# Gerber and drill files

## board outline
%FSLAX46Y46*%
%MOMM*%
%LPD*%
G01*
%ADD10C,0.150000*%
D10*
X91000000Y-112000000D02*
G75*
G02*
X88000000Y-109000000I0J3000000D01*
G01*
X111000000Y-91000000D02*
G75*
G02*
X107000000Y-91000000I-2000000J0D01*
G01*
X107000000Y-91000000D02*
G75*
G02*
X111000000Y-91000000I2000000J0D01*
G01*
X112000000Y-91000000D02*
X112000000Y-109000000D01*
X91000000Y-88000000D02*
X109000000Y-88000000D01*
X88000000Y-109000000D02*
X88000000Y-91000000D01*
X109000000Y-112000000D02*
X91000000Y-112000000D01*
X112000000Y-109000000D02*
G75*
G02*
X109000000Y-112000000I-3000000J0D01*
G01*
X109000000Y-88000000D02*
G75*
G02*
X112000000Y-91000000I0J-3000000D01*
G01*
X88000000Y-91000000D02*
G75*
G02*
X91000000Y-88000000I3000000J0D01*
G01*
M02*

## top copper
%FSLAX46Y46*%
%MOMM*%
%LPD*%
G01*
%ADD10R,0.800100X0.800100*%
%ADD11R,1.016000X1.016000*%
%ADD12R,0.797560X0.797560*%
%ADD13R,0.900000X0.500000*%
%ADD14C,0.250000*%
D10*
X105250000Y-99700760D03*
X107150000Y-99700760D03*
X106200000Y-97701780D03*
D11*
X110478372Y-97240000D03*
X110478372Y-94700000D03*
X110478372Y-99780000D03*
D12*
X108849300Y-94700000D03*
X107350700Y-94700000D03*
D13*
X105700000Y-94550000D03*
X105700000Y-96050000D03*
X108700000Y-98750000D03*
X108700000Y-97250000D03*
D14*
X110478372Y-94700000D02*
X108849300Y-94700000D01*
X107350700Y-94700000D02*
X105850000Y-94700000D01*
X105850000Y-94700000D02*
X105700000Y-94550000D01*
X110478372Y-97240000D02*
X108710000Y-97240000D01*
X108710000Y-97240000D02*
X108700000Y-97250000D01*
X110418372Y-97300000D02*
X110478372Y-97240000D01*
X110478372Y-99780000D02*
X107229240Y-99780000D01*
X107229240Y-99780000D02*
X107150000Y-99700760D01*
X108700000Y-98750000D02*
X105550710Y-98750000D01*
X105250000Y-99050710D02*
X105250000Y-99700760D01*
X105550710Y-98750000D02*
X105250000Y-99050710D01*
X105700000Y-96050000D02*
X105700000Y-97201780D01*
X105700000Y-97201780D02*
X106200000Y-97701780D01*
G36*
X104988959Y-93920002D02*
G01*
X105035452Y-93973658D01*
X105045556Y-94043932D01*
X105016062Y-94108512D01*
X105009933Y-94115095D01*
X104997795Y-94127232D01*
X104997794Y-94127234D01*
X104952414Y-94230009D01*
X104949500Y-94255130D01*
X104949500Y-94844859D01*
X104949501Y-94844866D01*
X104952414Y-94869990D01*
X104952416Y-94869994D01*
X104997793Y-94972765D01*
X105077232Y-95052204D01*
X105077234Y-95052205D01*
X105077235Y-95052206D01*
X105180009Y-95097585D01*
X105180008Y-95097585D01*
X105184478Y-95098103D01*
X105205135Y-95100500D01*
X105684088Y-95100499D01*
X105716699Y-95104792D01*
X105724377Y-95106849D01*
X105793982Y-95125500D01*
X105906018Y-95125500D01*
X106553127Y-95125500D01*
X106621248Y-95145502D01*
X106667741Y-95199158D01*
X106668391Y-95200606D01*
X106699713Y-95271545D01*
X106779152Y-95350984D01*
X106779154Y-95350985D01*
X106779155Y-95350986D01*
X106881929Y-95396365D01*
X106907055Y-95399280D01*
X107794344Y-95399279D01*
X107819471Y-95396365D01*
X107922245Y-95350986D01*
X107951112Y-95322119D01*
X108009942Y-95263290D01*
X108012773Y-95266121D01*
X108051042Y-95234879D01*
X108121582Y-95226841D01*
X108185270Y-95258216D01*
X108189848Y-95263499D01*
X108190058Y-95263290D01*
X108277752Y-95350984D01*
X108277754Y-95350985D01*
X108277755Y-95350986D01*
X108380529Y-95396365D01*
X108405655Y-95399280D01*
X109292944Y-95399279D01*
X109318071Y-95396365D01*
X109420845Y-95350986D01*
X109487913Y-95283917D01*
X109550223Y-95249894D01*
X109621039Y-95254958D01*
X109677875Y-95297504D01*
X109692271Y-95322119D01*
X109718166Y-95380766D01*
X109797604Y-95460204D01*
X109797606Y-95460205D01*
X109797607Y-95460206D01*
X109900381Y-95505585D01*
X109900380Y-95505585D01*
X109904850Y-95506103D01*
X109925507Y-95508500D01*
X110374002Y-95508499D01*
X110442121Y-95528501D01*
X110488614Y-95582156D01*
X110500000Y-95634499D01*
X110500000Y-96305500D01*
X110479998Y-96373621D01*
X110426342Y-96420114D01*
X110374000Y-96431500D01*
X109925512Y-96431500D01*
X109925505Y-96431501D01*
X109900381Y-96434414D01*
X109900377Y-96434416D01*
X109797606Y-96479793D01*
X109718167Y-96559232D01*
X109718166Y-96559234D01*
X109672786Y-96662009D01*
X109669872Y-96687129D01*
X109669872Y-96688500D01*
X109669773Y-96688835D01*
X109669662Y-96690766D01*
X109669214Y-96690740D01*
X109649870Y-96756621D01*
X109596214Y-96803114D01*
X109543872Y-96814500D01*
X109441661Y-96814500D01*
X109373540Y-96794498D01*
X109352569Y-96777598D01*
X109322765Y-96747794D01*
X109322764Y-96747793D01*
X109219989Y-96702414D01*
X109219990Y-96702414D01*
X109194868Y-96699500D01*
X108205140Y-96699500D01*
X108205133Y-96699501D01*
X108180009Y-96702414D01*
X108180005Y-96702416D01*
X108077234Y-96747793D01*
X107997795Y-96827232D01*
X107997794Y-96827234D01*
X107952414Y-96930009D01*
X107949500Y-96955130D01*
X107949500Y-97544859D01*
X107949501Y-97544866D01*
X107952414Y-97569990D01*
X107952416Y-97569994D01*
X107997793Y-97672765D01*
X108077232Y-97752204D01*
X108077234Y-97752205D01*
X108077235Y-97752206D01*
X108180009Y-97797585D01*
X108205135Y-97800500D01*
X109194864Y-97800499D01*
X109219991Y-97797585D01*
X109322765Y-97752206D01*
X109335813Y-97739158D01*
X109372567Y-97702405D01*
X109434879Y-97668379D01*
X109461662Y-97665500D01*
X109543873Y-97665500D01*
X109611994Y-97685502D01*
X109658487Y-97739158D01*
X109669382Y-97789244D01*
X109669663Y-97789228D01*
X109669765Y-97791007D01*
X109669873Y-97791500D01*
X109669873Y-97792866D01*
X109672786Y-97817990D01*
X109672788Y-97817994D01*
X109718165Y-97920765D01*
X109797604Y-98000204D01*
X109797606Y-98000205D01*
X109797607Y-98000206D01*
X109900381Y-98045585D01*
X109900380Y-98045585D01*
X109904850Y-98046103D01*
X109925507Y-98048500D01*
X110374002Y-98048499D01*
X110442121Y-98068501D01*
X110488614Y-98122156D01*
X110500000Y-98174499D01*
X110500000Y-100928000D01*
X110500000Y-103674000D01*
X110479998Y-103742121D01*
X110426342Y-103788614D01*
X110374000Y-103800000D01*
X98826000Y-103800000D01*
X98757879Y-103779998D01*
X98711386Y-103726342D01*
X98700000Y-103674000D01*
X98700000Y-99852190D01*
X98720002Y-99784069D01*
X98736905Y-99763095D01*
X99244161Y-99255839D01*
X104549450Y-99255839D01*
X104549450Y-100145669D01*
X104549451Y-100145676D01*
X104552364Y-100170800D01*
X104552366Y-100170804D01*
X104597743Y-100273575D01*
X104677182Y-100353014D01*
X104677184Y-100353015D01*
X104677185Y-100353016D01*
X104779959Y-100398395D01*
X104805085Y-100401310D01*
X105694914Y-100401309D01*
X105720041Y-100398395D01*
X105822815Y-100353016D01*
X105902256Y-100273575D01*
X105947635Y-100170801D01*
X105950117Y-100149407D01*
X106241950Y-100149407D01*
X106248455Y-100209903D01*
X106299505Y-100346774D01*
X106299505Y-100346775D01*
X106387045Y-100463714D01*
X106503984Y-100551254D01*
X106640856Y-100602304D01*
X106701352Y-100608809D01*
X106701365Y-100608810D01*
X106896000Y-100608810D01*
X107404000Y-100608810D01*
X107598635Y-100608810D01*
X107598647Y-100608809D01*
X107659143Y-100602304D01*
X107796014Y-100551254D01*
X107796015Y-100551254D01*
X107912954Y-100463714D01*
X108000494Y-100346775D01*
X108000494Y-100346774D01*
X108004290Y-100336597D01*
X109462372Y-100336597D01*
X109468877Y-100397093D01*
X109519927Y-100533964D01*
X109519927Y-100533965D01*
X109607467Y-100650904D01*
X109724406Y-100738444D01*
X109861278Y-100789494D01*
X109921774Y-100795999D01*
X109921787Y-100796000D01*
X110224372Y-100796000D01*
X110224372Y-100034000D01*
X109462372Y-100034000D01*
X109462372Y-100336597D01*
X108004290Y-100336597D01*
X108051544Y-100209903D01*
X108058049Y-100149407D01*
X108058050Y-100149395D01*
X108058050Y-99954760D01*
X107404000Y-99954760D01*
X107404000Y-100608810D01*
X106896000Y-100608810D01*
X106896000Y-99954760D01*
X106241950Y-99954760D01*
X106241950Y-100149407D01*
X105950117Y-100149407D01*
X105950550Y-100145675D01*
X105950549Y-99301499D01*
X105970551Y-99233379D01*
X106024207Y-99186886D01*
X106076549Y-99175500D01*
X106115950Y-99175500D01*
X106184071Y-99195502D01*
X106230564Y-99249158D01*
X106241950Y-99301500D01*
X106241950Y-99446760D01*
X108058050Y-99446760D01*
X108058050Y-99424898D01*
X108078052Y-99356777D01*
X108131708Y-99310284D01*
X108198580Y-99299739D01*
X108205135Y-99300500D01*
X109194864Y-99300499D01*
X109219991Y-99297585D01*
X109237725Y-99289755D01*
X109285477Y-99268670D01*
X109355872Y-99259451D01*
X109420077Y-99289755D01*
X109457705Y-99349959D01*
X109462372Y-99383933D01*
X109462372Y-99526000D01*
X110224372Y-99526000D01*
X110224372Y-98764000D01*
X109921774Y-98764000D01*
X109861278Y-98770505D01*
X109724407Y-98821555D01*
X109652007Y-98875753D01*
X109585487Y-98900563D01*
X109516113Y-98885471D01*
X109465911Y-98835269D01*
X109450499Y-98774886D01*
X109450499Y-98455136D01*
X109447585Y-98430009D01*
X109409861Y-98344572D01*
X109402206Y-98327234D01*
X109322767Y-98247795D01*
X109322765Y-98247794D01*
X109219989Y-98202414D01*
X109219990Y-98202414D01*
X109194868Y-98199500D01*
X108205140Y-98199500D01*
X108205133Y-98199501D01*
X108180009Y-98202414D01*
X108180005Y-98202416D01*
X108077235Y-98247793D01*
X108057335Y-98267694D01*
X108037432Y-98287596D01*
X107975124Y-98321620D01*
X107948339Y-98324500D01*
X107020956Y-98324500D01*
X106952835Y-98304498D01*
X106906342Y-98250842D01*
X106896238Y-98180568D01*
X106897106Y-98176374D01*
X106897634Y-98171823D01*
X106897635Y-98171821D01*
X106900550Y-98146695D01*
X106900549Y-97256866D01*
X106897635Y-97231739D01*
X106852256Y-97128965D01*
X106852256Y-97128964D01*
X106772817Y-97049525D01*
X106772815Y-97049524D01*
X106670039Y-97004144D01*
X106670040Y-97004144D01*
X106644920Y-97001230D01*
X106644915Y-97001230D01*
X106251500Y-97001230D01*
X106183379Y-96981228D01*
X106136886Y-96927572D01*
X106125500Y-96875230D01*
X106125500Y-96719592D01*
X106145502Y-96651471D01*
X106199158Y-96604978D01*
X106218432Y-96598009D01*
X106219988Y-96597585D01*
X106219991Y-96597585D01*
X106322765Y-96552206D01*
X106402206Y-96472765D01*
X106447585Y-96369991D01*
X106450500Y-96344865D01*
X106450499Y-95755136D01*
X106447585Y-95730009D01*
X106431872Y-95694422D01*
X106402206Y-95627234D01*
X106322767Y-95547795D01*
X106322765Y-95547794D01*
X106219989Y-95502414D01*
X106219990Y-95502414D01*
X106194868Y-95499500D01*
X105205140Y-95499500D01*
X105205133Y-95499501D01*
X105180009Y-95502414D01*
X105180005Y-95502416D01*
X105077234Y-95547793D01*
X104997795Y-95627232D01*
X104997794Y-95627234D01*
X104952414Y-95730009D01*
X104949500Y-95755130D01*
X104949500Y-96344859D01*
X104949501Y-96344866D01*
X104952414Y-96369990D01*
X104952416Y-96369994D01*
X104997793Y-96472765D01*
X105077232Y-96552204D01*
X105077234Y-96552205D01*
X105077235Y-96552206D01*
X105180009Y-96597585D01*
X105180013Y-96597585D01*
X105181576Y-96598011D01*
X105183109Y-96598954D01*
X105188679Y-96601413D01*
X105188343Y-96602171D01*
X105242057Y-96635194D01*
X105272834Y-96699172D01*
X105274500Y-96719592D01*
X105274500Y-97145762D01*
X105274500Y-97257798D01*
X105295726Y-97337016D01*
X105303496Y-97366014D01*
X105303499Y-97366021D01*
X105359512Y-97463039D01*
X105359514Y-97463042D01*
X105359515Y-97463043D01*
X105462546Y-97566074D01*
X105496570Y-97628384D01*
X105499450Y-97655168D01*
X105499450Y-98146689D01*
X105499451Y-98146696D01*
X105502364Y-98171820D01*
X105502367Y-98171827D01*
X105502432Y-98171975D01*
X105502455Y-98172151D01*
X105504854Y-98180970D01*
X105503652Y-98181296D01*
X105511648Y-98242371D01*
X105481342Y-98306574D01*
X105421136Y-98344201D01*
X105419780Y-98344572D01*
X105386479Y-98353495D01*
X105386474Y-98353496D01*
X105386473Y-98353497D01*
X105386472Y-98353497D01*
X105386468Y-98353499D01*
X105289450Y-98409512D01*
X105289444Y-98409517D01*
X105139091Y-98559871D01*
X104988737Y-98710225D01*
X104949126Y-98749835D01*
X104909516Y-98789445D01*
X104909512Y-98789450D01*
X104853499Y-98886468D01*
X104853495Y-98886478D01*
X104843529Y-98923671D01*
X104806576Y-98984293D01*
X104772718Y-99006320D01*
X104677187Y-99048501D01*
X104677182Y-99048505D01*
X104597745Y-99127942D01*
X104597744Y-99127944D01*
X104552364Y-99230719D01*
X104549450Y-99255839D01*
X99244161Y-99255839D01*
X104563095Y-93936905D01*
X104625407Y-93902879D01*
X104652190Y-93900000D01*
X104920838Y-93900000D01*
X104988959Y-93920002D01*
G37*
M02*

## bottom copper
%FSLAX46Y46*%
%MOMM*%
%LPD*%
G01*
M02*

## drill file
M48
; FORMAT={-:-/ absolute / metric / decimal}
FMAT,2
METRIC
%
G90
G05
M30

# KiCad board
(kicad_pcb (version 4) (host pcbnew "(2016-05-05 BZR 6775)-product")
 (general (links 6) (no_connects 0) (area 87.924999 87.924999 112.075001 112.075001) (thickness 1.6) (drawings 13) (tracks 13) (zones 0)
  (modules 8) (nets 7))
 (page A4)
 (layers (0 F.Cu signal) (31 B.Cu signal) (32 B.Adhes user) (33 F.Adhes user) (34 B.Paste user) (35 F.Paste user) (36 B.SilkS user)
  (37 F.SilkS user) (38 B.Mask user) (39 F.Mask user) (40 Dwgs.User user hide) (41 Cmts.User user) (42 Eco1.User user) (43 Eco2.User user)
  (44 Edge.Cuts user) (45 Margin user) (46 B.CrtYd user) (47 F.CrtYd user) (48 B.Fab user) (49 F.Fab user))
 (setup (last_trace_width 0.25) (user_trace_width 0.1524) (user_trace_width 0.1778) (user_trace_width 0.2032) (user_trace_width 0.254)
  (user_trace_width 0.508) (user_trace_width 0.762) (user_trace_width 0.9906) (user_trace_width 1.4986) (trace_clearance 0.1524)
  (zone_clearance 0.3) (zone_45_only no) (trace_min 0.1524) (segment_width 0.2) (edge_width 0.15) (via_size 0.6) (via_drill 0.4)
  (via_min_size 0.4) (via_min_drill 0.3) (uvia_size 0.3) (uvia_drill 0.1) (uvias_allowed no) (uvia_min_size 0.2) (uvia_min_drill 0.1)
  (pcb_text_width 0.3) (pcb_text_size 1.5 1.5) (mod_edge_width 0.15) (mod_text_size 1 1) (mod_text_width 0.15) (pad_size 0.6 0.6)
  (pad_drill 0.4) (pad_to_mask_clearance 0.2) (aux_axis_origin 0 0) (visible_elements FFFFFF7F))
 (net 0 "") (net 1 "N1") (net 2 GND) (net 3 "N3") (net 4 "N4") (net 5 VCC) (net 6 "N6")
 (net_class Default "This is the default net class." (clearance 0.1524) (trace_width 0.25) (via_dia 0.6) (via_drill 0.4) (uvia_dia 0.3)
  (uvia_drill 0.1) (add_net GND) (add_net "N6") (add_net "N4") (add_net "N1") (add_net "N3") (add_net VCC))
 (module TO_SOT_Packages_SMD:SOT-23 (layer F.Cu) (at 106.2 98.7)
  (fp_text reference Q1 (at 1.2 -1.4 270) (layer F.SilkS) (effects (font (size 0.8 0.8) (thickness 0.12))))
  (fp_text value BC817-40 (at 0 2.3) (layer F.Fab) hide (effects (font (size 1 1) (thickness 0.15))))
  (pad 1 smd rect (at -0.95 1.00076) (size 0.8001 0.8001) (layers F.Cu F.Paste F.Mask) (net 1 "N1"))
  (pad 2 smd rect (at 0.95 1.00076) (size 0.8001 0.8001) (layers F.Cu F.Paste F.Mask) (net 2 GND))
  (pad 3 smd rect (at 0 -0.99822) (size 0.8001 0.8001) (layers F.Cu F.Paste F.Mask) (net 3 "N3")))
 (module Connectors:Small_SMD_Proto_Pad (layer F.Cu) (at 110.478372 97.24 180)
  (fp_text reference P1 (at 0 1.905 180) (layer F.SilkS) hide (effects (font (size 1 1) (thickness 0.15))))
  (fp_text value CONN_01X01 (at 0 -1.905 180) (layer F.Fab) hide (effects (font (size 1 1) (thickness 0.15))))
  (pad 1 smd rect (at 0 0 180) (size 1.016 1.016) (layers F.Cu F.Paste F.Mask) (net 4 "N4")))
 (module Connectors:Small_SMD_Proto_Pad (layer F.Cu) (at 110.478372 94.7 180)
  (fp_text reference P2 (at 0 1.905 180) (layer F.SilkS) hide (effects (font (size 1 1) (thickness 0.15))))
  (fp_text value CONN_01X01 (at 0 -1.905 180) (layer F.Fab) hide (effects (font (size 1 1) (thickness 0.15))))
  (pad 1 smd rect (at 0 0 180) (size 1.016 1.016) (layers F.Cu F.Paste F.Mask) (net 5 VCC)))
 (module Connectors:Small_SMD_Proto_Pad (layer F.Cu) (at 110.478372 99.78 180)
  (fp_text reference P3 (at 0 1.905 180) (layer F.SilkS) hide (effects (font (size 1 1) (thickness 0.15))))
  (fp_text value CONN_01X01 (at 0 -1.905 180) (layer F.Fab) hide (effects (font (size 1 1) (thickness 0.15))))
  (pad 1 smd rect (at 0 0 180) (size 1.016 1.016) (layers F.Cu F.Paste F.Mask) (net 2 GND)))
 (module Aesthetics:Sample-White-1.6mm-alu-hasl (layer F.Cu) (at 99.978372 102.6)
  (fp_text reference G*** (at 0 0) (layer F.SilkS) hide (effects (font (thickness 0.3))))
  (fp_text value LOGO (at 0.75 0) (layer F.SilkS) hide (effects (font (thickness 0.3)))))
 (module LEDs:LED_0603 (layer F.Cu) (at 108.1 94.7)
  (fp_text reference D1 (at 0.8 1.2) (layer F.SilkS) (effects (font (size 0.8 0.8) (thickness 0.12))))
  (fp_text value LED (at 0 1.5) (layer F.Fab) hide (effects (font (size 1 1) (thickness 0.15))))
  (pad 2 smd rect (at 0.7493 0 180) (size 0.79756 0.79756) (layers F.Cu F.Paste F.Mask) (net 5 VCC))
  (pad 1 smd rect (at -0.7493 0 180) (size 0.79756 0.79756) (layers F.Cu F.Paste F.Mask) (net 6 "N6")))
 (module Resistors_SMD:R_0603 (layer F.Cu) (at 105.7 95.3 270)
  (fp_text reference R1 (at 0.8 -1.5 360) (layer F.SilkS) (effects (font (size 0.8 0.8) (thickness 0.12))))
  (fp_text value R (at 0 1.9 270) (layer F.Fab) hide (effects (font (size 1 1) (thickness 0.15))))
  (pad 1 smd rect (at -0.75 0 270) (size 0.5 0.9) (layers F.Cu F.Paste F.Mask) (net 6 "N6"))
  (pad 2 smd rect (at 0.75 0 270) (size 0.5 0.9) (layers F.Cu F.Paste F.Mask) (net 3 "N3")))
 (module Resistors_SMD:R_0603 (layer F.Cu) (at 108.7 98 90)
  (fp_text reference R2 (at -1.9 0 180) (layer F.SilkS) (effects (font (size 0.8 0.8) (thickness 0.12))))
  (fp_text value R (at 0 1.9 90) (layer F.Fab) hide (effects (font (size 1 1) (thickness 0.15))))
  (pad 1 smd rect (at -0.75 0 90) (size 0.5 0.9) (layers F.Cu F.Paste F.Mask) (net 1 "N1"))
  (pad 2 smd rect (at 0.75 0 90) (size 0.5 0.9) (layers F.Cu F.Paste F.Mask) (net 4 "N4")))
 (gr_arc (start 91 109) (end 91 112) (angle 90) (layer Edge.Cuts) (width 0.15))
 (gr_circle (center 109 91) (end 111 91) (layer Edge.Cuts) (width 0.15))
 (gr_line (start 112 91) (end 112 109) (layer Edge.Cuts) (width 0.15))
 (gr_line (start 91 88) (end 109 88) (layer Edge.Cuts) (width 0.15))
 (gr_line (start 88 109) (end 88 91) (layer Edge.Cuts) (width 0.15))
 (gr_line (start 109 112) (end 91 112) (layer Edge.Cuts) (width 0.15))
 (gr_arc (start 109 109) (end 112 109) (angle 90) (layer Edge.Cuts) (width 0.15))
 (gr_arc (start 109 91) (end 109 88) (angle 90) (layer Edge.Cuts) (width 0.15))
 (gr_arc (start 91 91) (end 88 91) (angle 90) (layer Edge.Cuts) (width 0.15))
 (segment (start 110.478372 94.7) (end 108.8493 94.7) (width 0.25) (layer F.Cu) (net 5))
 (segment (start 107.3507 94.7) (end 105.85 94.7) (width 0.25) (layer F.Cu) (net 6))
 (segment (start 105.85 94.7) (end 105.7 94.55) (width 0.25) (layer F.Cu) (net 6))
 (segment (start 110.478372 97.24) (end 108.71 97.24) (width 0.25) (layer F.Cu) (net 4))
 (segment (start 108.71 97.24) (end 108.7 97.25) (width 0.25) (layer F.Cu) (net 4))
 (segment (start 110.418372 97.3) (end 110.478372 97.24) (width 0.25) (layer F.Cu) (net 4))
 (segment (start 110.478372 99.78) (end 107.22924 99.78) (width 0.25) (layer F.Cu) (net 2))
 (segment (start 107.22924 99.78) (end 107.15 99.70076) (width 0.25) (layer F.Cu) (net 2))
 (segment (start 108.7 98.75) (end 105.55071 98.75) (width 0.25) (layer F.Cu) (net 1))
 (segment (start 105.25 99.05071) (end 105.25 99.70076) (width 0.25) (layer F.Cu) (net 1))
 (segment (start 105.55071 98.75) (end 105.25 99.05071) (width 0.25) (layer F.Cu) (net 1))
 (segment (start 105.7 96.05) (end 105.7 97.20178) (width 0.25) (layer F.Cu) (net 3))
 (segment (start 105.7 97.20178) (end 106.2 97.70178) (width 0.25) (layer F.Cu) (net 3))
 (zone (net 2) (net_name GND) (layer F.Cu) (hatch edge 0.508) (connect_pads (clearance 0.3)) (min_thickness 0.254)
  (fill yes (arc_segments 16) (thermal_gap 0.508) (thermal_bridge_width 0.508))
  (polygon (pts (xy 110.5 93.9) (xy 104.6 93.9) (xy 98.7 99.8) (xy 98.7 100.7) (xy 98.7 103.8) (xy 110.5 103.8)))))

